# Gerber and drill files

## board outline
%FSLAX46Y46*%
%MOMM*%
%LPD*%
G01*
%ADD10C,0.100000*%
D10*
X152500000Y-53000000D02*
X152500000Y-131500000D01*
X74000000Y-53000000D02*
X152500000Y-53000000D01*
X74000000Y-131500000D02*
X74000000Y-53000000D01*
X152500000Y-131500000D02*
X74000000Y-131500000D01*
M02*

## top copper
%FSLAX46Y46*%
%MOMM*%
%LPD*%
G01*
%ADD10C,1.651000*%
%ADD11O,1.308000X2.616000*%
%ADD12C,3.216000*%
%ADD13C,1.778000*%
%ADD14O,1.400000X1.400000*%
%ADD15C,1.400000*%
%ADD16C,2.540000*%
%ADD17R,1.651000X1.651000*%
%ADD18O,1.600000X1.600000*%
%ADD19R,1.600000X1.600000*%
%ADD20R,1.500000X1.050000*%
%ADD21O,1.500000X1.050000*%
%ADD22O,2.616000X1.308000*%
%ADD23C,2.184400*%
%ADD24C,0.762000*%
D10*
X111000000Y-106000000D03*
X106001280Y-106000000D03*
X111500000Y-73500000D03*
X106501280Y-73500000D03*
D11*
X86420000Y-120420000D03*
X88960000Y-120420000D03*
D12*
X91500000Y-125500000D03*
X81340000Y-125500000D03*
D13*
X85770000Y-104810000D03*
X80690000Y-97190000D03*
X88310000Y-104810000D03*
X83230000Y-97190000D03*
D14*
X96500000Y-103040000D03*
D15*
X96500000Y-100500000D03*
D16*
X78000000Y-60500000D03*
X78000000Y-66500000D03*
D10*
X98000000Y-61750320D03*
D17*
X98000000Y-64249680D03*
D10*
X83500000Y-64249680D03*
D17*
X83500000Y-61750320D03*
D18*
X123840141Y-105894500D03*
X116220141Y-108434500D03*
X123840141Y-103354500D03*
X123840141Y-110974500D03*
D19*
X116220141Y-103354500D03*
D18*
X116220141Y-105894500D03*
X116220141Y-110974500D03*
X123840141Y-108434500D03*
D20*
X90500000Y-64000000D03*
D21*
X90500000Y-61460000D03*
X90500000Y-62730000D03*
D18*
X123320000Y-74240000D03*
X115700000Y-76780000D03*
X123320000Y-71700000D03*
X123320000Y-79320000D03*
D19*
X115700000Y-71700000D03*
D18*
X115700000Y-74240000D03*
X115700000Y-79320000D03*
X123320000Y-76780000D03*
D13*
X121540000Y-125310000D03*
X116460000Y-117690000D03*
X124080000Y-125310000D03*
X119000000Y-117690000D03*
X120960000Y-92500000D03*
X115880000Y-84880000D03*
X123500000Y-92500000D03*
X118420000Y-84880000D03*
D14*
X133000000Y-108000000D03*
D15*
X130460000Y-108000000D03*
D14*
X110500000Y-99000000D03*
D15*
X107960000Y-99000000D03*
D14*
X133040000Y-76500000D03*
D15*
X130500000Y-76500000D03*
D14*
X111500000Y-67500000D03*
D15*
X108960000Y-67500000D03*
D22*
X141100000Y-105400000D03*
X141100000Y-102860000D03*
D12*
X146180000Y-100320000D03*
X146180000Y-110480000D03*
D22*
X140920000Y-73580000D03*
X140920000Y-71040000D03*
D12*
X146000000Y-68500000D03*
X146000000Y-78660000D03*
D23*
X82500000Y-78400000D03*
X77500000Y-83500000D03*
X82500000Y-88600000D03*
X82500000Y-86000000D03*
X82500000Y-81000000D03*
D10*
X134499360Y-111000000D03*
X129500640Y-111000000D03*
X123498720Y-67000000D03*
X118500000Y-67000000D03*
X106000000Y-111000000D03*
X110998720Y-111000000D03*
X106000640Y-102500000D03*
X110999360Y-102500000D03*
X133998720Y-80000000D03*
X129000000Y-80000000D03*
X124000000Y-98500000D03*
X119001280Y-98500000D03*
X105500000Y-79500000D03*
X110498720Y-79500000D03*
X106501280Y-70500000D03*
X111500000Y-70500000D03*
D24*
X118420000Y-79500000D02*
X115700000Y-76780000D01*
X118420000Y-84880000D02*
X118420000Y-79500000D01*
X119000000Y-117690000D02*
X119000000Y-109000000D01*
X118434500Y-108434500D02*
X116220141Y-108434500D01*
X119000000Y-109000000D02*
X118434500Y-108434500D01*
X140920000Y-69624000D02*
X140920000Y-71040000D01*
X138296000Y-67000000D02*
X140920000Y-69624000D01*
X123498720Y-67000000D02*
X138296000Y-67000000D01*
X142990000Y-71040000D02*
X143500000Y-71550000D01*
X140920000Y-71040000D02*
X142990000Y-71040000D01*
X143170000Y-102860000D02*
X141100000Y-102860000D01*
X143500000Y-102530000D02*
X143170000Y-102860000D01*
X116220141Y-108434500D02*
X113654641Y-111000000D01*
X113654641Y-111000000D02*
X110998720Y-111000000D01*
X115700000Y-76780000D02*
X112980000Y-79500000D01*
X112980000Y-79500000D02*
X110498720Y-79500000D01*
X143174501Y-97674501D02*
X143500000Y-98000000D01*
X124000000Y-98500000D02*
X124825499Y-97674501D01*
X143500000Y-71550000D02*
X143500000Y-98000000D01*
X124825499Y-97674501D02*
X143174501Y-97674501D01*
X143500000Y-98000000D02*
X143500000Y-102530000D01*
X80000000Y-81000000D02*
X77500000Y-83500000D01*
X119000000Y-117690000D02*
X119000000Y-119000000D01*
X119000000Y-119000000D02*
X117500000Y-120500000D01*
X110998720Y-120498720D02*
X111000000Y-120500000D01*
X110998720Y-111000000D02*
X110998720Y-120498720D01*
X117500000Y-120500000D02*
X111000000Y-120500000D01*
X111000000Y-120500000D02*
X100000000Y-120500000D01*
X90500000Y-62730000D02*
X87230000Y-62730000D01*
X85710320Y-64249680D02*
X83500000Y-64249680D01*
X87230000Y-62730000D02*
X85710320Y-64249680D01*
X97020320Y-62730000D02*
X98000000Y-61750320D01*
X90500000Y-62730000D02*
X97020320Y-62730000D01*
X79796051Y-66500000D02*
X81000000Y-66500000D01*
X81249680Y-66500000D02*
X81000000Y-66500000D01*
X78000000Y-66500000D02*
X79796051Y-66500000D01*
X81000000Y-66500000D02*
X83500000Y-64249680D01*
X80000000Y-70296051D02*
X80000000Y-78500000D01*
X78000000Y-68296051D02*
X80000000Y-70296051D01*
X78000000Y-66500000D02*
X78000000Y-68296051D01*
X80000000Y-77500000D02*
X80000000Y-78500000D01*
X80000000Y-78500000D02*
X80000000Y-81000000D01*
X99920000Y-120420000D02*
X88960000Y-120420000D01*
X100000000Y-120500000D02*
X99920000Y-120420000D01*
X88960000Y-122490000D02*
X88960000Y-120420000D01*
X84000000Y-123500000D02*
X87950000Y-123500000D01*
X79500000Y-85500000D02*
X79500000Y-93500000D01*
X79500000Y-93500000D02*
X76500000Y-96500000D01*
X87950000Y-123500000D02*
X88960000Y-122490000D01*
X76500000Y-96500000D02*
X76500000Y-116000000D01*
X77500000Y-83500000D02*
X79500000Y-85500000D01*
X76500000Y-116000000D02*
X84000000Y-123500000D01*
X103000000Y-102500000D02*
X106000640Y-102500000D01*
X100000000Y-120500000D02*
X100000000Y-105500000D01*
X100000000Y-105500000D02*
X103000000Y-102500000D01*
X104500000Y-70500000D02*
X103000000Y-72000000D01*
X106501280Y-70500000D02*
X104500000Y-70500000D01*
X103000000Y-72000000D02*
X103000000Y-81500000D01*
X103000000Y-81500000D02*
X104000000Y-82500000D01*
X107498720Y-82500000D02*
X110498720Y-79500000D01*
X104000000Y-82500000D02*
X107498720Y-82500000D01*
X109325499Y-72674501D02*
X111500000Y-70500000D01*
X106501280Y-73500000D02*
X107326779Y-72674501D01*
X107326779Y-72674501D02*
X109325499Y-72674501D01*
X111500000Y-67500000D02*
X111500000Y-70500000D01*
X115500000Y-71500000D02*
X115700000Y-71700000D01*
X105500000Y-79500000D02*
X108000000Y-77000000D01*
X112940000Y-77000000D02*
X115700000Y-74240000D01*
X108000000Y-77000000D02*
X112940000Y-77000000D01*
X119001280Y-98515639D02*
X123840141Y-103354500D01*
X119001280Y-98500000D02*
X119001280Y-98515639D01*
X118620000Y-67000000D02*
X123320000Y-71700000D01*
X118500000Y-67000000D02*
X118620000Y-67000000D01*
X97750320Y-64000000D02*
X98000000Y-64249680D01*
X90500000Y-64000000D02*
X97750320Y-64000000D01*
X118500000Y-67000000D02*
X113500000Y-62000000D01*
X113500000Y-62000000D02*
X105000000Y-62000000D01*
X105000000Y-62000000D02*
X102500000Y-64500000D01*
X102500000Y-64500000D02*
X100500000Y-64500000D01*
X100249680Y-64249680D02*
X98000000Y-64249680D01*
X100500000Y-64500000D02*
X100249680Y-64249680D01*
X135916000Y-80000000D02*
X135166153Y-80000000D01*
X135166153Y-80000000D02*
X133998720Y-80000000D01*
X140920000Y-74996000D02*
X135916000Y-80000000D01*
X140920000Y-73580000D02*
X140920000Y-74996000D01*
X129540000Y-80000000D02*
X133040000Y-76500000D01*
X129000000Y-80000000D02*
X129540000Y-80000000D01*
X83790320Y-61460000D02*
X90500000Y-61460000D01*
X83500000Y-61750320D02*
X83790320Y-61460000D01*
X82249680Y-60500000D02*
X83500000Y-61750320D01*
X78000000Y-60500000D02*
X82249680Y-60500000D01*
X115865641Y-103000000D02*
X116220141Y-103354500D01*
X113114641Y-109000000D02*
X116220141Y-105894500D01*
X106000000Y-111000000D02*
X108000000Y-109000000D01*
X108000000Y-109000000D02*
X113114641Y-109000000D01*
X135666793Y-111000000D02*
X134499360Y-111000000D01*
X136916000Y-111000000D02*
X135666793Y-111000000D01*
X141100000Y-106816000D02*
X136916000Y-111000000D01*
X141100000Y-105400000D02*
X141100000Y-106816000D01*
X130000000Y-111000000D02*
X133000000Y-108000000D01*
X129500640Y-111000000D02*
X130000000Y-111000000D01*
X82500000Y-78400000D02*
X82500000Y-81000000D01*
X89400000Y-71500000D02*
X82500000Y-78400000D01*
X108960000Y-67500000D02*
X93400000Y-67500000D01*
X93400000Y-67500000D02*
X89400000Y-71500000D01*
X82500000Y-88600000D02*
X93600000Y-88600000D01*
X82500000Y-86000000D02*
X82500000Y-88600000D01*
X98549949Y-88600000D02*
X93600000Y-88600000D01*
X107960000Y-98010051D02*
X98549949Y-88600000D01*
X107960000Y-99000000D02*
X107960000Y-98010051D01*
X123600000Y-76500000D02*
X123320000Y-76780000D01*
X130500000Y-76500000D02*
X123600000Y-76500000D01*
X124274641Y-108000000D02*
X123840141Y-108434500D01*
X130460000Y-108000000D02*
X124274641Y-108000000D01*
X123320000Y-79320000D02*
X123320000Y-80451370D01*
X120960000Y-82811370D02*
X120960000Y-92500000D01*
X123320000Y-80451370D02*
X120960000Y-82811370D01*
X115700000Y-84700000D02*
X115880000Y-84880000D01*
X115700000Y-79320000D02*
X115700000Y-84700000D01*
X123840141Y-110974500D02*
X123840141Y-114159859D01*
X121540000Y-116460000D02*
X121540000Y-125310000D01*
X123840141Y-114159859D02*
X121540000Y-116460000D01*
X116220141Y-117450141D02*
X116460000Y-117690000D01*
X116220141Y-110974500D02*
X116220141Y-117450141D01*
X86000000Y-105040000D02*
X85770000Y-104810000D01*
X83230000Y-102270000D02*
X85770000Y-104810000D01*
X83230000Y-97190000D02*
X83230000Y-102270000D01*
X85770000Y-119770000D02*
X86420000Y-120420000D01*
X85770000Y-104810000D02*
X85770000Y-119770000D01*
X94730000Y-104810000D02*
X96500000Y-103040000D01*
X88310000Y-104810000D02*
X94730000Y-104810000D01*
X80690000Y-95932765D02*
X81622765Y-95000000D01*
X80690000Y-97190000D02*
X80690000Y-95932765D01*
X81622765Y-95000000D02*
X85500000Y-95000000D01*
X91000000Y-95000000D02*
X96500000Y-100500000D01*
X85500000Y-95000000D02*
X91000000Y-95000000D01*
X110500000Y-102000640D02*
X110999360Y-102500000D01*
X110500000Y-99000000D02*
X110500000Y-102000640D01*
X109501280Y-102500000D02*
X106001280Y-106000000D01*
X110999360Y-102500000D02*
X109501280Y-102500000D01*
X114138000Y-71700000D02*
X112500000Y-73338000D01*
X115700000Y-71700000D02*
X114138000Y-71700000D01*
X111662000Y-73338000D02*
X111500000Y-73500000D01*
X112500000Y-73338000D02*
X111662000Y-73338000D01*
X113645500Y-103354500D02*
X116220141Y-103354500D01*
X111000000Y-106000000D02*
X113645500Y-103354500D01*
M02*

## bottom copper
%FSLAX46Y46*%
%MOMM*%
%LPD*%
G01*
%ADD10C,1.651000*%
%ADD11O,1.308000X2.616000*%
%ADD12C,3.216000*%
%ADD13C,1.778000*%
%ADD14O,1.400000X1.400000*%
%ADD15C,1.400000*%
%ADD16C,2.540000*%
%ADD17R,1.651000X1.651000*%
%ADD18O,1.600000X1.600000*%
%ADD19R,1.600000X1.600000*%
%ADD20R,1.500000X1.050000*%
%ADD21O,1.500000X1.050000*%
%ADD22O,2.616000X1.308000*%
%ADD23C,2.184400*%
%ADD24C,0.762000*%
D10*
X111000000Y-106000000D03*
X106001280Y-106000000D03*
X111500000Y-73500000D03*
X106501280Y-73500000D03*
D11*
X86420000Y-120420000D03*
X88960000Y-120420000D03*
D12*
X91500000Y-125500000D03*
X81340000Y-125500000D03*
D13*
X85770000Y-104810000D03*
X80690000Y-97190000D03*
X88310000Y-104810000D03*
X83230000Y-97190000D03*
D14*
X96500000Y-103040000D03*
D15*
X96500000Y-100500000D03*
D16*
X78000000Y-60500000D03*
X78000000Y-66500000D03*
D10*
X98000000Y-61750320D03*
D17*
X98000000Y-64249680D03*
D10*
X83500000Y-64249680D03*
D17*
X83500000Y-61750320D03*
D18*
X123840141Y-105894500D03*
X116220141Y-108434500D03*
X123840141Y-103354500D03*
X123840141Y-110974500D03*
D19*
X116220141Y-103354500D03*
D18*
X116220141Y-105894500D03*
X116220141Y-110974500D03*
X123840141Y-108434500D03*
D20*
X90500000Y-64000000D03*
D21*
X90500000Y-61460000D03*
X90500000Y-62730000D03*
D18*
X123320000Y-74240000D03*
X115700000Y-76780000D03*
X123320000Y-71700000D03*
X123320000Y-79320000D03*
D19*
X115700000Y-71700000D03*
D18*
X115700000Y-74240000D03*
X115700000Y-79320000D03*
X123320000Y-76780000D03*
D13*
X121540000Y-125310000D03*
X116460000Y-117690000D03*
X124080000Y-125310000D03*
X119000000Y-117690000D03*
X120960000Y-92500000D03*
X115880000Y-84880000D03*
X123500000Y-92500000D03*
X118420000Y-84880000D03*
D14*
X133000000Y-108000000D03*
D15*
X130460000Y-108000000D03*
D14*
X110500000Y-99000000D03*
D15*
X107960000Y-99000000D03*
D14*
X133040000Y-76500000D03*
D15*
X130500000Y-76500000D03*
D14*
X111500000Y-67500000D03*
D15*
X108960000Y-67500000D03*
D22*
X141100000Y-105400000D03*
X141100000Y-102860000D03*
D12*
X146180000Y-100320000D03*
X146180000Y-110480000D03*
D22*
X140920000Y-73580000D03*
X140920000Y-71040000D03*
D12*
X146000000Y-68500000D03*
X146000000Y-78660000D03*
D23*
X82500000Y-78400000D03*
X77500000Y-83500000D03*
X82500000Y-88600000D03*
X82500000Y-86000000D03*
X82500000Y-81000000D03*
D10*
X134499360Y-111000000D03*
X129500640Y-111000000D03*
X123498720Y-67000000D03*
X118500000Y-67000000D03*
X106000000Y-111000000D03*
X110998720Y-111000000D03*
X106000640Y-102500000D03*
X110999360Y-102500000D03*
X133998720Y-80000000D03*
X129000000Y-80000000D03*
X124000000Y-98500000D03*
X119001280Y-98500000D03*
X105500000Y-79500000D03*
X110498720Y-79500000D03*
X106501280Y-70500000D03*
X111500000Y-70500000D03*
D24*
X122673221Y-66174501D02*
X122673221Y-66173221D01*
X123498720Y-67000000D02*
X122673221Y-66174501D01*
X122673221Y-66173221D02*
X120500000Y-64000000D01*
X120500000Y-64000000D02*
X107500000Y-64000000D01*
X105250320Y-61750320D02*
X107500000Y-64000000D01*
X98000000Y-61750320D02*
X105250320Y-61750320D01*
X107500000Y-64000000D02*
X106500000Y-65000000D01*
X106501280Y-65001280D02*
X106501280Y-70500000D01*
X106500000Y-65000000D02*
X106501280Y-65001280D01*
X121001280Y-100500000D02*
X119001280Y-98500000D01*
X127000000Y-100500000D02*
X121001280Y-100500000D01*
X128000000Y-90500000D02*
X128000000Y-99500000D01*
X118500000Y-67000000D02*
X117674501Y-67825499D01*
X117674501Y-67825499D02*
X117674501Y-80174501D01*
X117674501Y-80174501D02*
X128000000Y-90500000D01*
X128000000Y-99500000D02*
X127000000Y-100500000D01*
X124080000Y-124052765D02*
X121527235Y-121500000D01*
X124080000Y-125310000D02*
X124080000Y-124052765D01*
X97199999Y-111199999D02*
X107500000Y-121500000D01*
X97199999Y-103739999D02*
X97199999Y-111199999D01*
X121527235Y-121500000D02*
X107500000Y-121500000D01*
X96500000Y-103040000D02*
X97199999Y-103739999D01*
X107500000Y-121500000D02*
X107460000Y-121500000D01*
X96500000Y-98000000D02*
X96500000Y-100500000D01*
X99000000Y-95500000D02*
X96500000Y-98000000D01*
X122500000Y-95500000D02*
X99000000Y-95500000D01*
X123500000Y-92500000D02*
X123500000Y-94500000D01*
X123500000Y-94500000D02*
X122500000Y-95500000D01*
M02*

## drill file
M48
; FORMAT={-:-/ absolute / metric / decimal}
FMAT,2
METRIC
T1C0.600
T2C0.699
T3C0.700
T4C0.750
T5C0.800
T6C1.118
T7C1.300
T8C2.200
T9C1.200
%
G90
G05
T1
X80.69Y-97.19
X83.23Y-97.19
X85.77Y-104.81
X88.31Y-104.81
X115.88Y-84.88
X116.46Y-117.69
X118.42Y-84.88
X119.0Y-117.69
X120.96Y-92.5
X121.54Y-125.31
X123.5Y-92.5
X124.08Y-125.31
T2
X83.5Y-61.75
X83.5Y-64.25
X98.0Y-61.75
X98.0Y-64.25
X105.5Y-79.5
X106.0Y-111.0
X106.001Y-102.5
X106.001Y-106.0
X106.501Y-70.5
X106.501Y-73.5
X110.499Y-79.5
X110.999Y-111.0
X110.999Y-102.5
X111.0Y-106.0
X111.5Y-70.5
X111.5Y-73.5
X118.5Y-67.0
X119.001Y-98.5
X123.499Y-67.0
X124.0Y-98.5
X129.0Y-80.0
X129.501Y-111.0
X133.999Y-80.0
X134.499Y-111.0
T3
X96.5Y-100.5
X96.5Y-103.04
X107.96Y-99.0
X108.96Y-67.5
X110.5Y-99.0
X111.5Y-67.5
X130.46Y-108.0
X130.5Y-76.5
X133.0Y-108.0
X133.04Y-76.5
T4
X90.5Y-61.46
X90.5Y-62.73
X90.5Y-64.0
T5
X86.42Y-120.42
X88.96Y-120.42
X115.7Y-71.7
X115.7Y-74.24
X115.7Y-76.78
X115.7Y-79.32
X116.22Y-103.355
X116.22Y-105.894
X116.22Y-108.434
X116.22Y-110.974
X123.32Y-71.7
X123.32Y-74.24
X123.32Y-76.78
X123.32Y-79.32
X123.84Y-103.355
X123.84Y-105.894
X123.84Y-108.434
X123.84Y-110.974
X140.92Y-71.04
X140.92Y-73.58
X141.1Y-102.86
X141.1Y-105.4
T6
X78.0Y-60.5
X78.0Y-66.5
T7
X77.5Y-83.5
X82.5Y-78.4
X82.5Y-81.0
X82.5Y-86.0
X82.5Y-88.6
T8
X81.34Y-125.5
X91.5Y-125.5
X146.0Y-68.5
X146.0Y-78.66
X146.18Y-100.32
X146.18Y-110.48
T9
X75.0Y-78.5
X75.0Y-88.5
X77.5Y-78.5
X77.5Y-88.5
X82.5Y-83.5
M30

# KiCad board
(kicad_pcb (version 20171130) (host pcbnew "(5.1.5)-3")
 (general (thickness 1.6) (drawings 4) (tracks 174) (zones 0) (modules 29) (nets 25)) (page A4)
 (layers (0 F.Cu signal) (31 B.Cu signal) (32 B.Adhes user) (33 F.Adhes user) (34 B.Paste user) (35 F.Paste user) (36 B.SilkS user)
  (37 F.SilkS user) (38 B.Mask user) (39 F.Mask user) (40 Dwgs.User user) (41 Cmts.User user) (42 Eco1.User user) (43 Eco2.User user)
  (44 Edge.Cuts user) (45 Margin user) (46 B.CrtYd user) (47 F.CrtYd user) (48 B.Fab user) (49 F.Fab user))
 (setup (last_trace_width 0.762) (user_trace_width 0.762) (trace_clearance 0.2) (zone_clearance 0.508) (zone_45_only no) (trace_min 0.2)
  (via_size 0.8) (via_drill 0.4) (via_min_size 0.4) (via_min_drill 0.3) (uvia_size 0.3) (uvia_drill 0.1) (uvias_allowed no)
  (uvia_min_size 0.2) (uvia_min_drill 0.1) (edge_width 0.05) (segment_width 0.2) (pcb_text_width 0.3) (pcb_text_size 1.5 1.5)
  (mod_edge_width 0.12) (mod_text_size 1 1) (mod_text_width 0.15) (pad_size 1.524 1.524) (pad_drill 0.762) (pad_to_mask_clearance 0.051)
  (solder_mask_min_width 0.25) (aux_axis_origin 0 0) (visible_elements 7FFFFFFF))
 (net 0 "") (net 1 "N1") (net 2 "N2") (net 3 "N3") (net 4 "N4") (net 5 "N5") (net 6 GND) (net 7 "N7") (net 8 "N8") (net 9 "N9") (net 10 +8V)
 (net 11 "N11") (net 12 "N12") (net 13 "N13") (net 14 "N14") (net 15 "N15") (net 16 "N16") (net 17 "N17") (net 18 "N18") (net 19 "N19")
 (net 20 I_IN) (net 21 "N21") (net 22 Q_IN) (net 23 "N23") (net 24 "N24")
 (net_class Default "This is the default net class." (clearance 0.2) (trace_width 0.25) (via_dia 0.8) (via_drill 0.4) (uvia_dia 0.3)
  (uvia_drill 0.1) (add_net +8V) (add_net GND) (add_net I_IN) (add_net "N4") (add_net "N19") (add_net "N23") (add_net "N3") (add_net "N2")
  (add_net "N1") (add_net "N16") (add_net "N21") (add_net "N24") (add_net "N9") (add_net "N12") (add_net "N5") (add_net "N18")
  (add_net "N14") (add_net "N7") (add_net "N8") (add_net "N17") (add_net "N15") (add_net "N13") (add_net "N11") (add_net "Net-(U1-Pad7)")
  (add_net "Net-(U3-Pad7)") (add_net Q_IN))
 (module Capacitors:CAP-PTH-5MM (layer F.Cu) (at 108.50064 106)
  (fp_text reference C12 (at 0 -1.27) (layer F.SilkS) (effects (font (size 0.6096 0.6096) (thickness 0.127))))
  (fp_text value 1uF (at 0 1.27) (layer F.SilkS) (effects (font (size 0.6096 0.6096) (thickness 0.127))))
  (pad 2 thru_hole circle (at 2.49936 0) (size 1.651 1.651) (drill 0.6985) (layers *.Cu *.Mask) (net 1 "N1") (solder_mask_margin 0.1016))
  (pad 1 thru_hole circle (at -2.49936 0) (size 1.651 1.651) (drill 0.6985) (layers *.Cu *.Mask) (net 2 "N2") (solder_mask_margin 0.1016)))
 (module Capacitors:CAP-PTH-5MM (layer F.Cu) (at 109.00064 73.5)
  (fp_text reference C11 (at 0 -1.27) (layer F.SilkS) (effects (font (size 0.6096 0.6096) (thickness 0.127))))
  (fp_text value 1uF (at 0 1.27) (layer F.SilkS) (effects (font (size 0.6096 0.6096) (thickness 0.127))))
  (pad 2 thru_hole circle (at 2.49936 0) (size 1.651 1.651) (drill 0.6985) (layers *.Cu *.Mask) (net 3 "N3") (solder_mask_margin 0.1016))
  (pad 1 thru_hole circle (at -2.49936 0) (size 1.651 1.651) (drill 0.6985) (layers *.Cu *.Mask) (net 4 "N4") (solder_mask_margin 0.1016)))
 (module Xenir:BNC (layer F.Cu) (at 86.32 124.32 180)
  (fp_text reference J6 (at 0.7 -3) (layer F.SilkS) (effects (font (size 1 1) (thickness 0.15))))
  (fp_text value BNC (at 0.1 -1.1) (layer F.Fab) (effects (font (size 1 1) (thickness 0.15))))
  (pad S thru_hole oval (at -0.1 3.9 270) (size 2.616 1.308) (drill 0.8) (layers *.Cu *.Mask) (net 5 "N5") (solder_mask_margin 0.1016))
  (pad GND thru_hole oval (at -2.64 3.9 270) (size 2.616 1.308) (drill 0.8) (layers *.Cu *.Mask) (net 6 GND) (solder_mask_margin 0.1016))
  (pad 3 thru_hole circle (at -5.18 -1.18 180) (size 3.216 3.216) (drill 2.2) (layers *.Cu *.Mask) (solder_mask_margin 0.1016))
  (pad 4 thru_hole circle (at 4.98 -1.18 180) (size 3.216 3.216) (drill 2.2) (layers *.Cu *.Mask) (solder_mask_margin 0.1016)))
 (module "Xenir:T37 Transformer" (layer F.Cu) (at 91.5 101 270)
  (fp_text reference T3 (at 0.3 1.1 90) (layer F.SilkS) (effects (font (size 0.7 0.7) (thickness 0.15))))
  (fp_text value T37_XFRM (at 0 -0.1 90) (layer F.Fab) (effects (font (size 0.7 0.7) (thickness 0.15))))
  (pad C1B thru_hole circle (at 3.81 5.73 270) (size 1.778 1.778) (drill 0.6) (layers *.Cu *.Mask) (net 5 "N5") (solder_mask_margin 0.1016))
  (pad C1A thru_hole circle (at -3.81 10.81 270) (size 1.778 1.778) (drill 0.6) (layers *.Cu *.Mask) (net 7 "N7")
   (solder_mask_margin 0.1016))
  (pad C2B thru_hole circle (at 3.81 3.19 270) (size 1.778 1.778) (drill 0.6) (layers *.Cu *.Mask) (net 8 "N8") (solder_mask_margin 0.1016))
  (pad C2A thru_hole circle (at -3.81 8.27 270) (size 1.778 1.778) (drill 0.6) (layers *.Cu *.Mask) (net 5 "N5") (solder_mask_margin 0.1016)))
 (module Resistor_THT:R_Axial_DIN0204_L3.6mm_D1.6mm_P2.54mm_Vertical (layer F.Cu) (at 96.5 100.5 270)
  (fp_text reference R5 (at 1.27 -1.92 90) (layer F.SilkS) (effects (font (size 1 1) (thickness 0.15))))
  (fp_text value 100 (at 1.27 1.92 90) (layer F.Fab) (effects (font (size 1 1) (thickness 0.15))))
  (pad 2 thru_hole oval (at 2.54 0 270) (size 1.4 1.4) (drill 0.7) (layers *.Cu *.Mask) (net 8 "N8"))
  (pad 1 thru_hole circle (at 0 0 270) (size 1.4 1.4) (drill 0.7) (layers *.Cu *.Mask) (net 7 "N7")))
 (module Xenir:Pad (layer F.Cu) (at 78 57)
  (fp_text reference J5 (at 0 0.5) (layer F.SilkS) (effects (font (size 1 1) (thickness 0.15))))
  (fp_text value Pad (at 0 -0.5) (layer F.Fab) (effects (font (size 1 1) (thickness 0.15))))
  (pad 1 thru_hole circle (at 0 3.5) (size 2.54 2.54) (drill 1.1176) (layers *.Cu *.Mask) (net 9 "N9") (solder_mask_margin 0.1016)))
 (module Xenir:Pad (layer F.Cu) (at 78 63)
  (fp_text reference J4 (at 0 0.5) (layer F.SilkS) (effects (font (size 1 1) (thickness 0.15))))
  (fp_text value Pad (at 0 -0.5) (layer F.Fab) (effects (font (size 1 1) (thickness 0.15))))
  (pad 1 thru_hole circle (at 0 3.5) (size 2.54 2.54) (drill 1.1176) (layers *.Cu *.Mask) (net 6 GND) (solder_mask_margin 0.1016)))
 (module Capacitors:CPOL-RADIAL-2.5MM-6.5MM (layer F.Cu) (at 98 63 270)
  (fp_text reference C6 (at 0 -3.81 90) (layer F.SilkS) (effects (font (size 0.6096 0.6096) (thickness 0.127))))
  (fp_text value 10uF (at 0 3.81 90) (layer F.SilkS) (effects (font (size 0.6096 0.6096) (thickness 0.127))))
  (pad 2 thru_hole circle (at -1.24968 0 270) (size 1.651 1.651) (drill 0.6985) (layers *.Cu *.Mask) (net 6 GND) (solder_mask_margin 0.1016))
  (pad 1 thru_hole rect (at 1.24968 0 270) (size 1.651 1.651) (drill 0.6985) (layers *.Cu *.Mask) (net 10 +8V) (solder_mask_margin 0.1016)))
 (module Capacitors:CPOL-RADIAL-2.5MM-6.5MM (layer F.Cu) (at 83.5 63 90)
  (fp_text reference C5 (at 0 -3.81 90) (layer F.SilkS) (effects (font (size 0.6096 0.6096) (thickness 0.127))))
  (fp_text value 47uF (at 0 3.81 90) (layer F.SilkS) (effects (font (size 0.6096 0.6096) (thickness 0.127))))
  (pad 2 thru_hole circle (at -1.24968 0 90) (size 1.651 1.651) (drill 0.6985) (layers *.Cu *.Mask) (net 6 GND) (solder_mask_margin 0.1016))
  (pad 1 thru_hole rect (at 1.24968 0 90) (size 1.651 1.651) (drill 0.6985) (layers *.Cu *.Mask) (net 9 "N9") (solder_mask_margin 0.1016)))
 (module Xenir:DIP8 (layer F.Cu) (at 120.020141 101.6545)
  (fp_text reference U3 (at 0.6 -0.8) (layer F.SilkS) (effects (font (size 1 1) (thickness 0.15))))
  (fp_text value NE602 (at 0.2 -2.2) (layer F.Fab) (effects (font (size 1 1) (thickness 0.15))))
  (pad 7 thru_hole oval (at 3.82 4.24) (size 1.6 1.6) (drill 0.8) (layers *.Cu *.Mask))
  (pad 3 thru_hole oval (at -3.8 6.78) (size 1.6 1.6) (drill 0.8) (layers *.Cu *.Mask) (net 6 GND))
  (pad 8 thru_hole oval (at 3.82 1.7) (size 1.6 1.6) (drill 0.8) (layers *.Cu *.Mask) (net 10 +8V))
  (pad 5 thru_hole oval (at 3.82 9.32) (size 1.6 1.6) (drill 0.8) (layers *.Cu *.Mask) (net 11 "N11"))
  (pad 1 thru_hole rect (at -3.8 1.7) (size 1.6 1.6) (drill 0.8) (layers *.Cu *.Mask) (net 1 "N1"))
  (pad 2 thru_hole oval (at -3.8 4.24) (size 1.6 1.6) (drill 0.8) (layers *.Cu *.Mask) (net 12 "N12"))
  (pad 4 thru_hole oval (at -3.8 9.32) (size 1.6 1.6) (drill 0.8) (layers *.Cu *.Mask) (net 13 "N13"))
  (pad 6 thru_hole oval (at 3.82 6.78) (size 1.6 1.6) (drill 0.8) (layers *.Cu *.Mask) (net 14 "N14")))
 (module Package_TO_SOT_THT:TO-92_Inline (layer F.Cu) (at 90.5 64 90)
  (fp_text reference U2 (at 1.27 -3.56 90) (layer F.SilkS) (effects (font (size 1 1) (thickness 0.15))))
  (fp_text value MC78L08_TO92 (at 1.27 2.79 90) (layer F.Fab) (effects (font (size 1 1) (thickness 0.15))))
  (pad 1 thru_hole rect (at 0 0 90) (size 1.05 1.5) (drill 0.75) (layers *.Cu *.Mask) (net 10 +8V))
  (pad 3 thru_hole oval (at 2.54 0 90) (size 1.05 1.5) (drill 0.75) (layers *.Cu *.Mask) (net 9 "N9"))
  (pad 2 thru_hole oval (at 1.27 0 90) (size 1.05 1.5) (drill 0.75) (layers *.Cu *.Mask) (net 6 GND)))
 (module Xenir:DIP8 (layer F.Cu) (at 119.5 70)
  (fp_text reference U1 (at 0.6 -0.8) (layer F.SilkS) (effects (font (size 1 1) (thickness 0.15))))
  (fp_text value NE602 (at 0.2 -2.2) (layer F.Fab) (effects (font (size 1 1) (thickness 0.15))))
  (pad 7 thru_hole oval (at 3.82 4.24) (size 1.6 1.6) (drill 0.8) (layers *.Cu *.Mask))
  (pad 3 thru_hole oval (at -3.8 6.78) (size 1.6 1.6) (drill 0.8) (layers *.Cu *.Mask) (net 6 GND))
  (pad 8 thru_hole oval (at 3.82 1.7) (size 1.6 1.6) (drill 0.8) (layers *.Cu *.Mask) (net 10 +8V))
  (pad 5 thru_hole oval (at 3.82 9.32) (size 1.6 1.6) (drill 0.8) (layers *.Cu *.Mask) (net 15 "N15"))
  (pad 1 thru_hole rect (at -3.8 1.7) (size 1.6 1.6) (drill 0.8) (layers *.Cu *.Mask) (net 3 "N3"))
  (pad 2 thru_hole oval (at -3.8 4.24) (size 1.6 1.6) (drill 0.8) (layers *.Cu *.Mask) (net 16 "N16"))
  (pad 4 thru_hole oval (at -3.8 9.32) (size 1.6 1.6) (drill 0.8) (layers *.Cu *.Mask) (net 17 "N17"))
  (pad 6 thru_hole oval (at 3.82 6.78) (size 1.6 1.6) (drill 0.8) (layers *.Cu *.Mask) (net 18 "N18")))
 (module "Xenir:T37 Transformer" (layer F.Cu) (at 127.27 121.5 270)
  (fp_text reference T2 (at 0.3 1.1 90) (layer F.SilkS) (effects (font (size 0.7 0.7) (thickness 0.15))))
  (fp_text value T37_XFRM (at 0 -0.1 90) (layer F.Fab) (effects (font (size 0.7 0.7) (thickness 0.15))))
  (pad C1B thru_hole circle (at 3.81 5.73 270) (size 1.778 1.778) (drill 0.6) (layers *.Cu *.Mask) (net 11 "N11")
   (solder_mask_margin 0.1016))
  (pad C1A thru_hole circle (at -3.81 10.81 270) (size 1.778 1.778) (drill 0.6) (layers *.Cu *.Mask) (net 13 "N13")
   (solder_mask_margin 0.1016))
  (pad C2B thru_hole circle (at 3.81 3.19 270) (size 1.778 1.778) (drill 0.6) (layers *.Cu *.Mask) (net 8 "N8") (solder_mask_margin 0.1016))
  (pad C2A thru_hole circle (at -3.81 8.27 270) (size 1.778 1.778) (drill 0.6) (layers *.Cu *.Mask) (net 6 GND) (solder_mask_margin 0.1016)))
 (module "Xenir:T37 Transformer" (layer F.Cu) (at 126.69 88.69 270)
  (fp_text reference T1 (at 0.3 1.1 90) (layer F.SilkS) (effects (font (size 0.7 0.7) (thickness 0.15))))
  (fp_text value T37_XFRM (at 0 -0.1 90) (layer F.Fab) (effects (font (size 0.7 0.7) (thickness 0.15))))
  (pad C1B thru_hole circle (at 3.81 5.73 270) (size 1.778 1.778) (drill 0.6) (layers *.Cu *.Mask) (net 15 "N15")
   (solder_mask_margin 0.1016))
  (pad C1A thru_hole circle (at -3.81 10.81 270) (size 1.778 1.778) (drill 0.6) (layers *.Cu *.Mask) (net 17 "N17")
   (solder_mask_margin 0.1016))
  (pad C2B thru_hole circle (at 3.81 3.19 270) (size 1.778 1.778) (drill 0.6) (layers *.Cu *.Mask) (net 7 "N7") (solder_mask_margin 0.1016))
  (pad C2A thru_hole circle (at -3.81 8.27 270) (size 1.778 1.778) (drill 0.6) (layers *.Cu *.Mask) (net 6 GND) (solder_mask_margin 0.1016)))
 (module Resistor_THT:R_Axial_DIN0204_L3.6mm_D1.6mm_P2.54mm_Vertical (layer F.Cu) (at 130.46 108)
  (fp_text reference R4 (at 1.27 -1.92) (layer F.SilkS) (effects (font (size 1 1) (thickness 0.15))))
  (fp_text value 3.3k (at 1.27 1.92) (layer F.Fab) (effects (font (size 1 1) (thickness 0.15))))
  (pad 2 thru_hole oval (at 2.54 0) (size 1.4 1.4) (drill 0.7) (layers *.Cu *.Mask) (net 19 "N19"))
  (pad 1 thru_hole circle (at 0 0) (size 1.4 1.4) (drill 0.7) (layers *.Cu *.Mask) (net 14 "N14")))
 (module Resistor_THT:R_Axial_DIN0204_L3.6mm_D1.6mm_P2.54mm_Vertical (layer F.Cu) (at 107.96 99)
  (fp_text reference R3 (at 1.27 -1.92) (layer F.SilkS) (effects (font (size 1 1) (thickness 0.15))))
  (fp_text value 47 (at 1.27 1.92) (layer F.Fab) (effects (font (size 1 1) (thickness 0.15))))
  (pad 2 thru_hole oval (at 2.54 0) (size 1.4 1.4) (drill 0.7) (layers *.Cu *.Mask) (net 2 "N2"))
  (pad 1 thru_hole circle (at 0 0) (size 1.4 1.4) (drill 0.7) (layers *.Cu *.Mask) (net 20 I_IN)))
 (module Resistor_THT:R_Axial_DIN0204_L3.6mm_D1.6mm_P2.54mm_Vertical (layer F.Cu) (at 130.5 76.5)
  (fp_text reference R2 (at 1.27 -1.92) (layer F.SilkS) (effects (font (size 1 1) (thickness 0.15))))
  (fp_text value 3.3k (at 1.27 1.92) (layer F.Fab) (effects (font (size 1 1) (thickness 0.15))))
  (pad 2 thru_hole oval (at 2.54 0) (size 1.4 1.4) (drill 0.7) (layers *.Cu *.Mask) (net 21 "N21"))
  (pad 1 thru_hole circle (at 0 0) (size 1.4 1.4) (drill 0.7) (layers *.Cu *.Mask) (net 18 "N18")))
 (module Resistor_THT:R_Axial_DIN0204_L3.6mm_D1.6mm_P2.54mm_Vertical (layer F.Cu) (at 108.96 67.5)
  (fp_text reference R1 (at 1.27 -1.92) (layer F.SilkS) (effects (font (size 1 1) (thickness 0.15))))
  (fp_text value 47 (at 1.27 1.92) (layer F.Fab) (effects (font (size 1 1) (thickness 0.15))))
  (pad 2 thru_hole oval (at 2.54 0) (size 1.4 1.4) (drill 0.7) (layers *.Cu *.Mask) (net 4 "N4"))
  (pad 1 thru_hole circle (at 0 0) (size 1.4 1.4) (drill 0.7) (layers *.Cu *.Mask) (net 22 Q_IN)))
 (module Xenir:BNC (layer F.Cu) (at 145 105.5 270)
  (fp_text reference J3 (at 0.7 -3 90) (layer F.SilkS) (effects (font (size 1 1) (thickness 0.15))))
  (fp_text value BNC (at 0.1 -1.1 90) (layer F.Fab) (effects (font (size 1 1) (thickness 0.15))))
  (pad S thru_hole oval (at -0.1 3.9) (size 2.616 1.308) (drill 0.8) (layers *.Cu *.Mask) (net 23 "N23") (solder_mask_margin 0.1016))
  (pad GND thru_hole oval (at -2.64 3.9) (size 2.616 1.308) (drill 0.8) (layers *.Cu *.Mask) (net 6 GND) (solder_mask_margin 0.1016))
  (pad 3 thru_hole circle (at -5.18 -1.18 270) (size 3.216 3.216) (drill 2.2) (layers *.Cu *.Mask) (solder_mask_margin 0.1016))
  (pad 4 thru_hole circle (at 4.98 -1.18 270) (size 3.216 3.216) (drill 2.2) (layers *.Cu *.Mask) (solder_mask_margin 0.1016)))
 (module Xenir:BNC (layer F.Cu) (at 144.82 73.68 270)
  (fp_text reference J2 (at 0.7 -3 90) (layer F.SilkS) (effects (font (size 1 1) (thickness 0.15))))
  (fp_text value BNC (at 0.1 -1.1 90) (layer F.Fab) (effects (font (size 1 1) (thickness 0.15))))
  (pad S thru_hole oval (at -0.1 3.9) (size 2.616 1.308) (drill 0.8) (layers *.Cu *.Mask) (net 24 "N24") (solder_mask_margin 0.1016))
  (pad GND thru_hole oval (at -2.64 3.9) (size 2.616 1.308) (drill 0.8) (layers *.Cu *.Mask) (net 6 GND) (solder_mask_margin 0.1016))
  (pad 3 thru_hole circle (at -5.18 -1.18 270) (size 3.216 3.216) (drill 2.2) (layers *.Cu *.Mask) (solder_mask_margin 0.1016))
  (pad 4 thru_hole circle (at 4.98 -1.18 270) (size 3.216 3.216) (drill 2.2) (layers *.Cu *.Mask) (solder_mask_margin 0.1016)))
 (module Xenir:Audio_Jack (layer F.Cu) (at 79.5 75)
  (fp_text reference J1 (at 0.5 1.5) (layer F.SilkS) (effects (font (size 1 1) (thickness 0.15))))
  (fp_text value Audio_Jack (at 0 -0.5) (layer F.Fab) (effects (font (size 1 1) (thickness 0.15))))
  (pad "" np_thru_hole circle (at -4.5 3.5) (size 1.2 1.2) (drill 1.2) (layers *.Cu *.Mask))
  (pad "" np_thru_hole circle (at -2 3.5) (size 1.2 1.2) (drill 1.2) (layers *.Cu *.Mask))
  (pad RING thru_hole circle (at 3 3.4) (size 2.1844 2.1844) (drill 1.3) (layers *.Cu *.Mask) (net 22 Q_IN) (solder_mask_margin 0.1016))
  (pad "" np_thru_hole circle (at 3 8.5) (size 1.2 1.2) (drill 1.2) (layers *.Cu *.Mask))
  (pad SLEEVE thru_hole circle (at -2 8.5) (size 2.1844 2.1844) (drill 1.3) (layers *.Cu *.Mask) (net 6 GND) (solder_mask_margin 0.1016))
  (pad "" np_thru_hole circle (at -2 13.5) (size 1.2 1.2) (drill 1.2) (layers *.Cu *.Mask))
  (pad TIP thru_hole circle (at 3 13.6) (size 2.1844 2.1844) (drill 1.3) (layers *.Cu *.Mask) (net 20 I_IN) (solder_mask_margin 0.1016))
  (pad TSH thru_hole circle (at 3 11) (size 2.1844 2.1844) (drill 1.3) (layers *.Cu *.Mask) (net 20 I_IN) (solder_mask_margin 0.1016))
  (pad "" np_thru_hole circle (at -4.5 13.5) (size 1.2 1.2) (drill 1.2) (layers *.Cu *.Mask))
  (pad RSH thru_hole circle (at 3 6) (size 2.1844 2.1844) (drill 1.3) (layers *.Cu *.Mask) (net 22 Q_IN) (solder_mask_margin 0.1016)))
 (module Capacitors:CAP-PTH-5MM (layer F.Cu) (at 132 111)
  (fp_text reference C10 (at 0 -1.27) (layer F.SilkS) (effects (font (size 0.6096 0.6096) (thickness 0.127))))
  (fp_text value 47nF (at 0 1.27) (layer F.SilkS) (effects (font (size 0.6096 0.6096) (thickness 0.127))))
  (pad 2 thru_hole circle (at 2.49936 0) (size 1.651 1.651) (drill 0.6985) (layers *.Cu *.Mask) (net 23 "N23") (solder_mask_margin 0.1016))
  (pad 1 thru_hole circle (at -2.49936 0) (size 1.651 1.651) (drill 0.6985) (layers *.Cu *.Mask) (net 19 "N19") (solder_mask_margin 0.1016)))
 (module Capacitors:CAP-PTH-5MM (layer F.Cu) (at 120.99936 67)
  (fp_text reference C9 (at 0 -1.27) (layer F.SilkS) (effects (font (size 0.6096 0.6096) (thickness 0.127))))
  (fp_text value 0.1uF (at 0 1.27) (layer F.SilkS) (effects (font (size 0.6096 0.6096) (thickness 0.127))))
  (pad 2 thru_hole circle (at 2.49936 0) (size 1.651 1.651) (drill 0.6985) (layers *.Cu *.Mask) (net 6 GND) (solder_mask_margin 0.1016))
  (pad 1 thru_hole circle (at -2.49936 0) (size 1.651 1.651) (drill 0.6985) (layers *.Cu *.Mask) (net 10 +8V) (solder_mask_margin 0.1016)))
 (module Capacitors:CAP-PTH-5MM (layer F.Cu) (at 108.49936 111 180)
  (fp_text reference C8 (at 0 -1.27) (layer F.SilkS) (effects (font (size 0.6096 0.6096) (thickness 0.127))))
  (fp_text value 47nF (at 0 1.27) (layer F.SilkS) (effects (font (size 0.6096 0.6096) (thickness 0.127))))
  (pad 2 thru_hole circle (at 2.49936 0 180) (size 1.651 1.651) (drill 0.6985) (layers *.Cu *.Mask) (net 12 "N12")
   (solder_mask_margin 0.1016))
  (pad 1 thru_hole circle (at -2.49936 0 180) (size 1.651 1.651) (drill 0.6985) (layers *.Cu *.Mask) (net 6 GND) (solder_mask_margin 0.1016)))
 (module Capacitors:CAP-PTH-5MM (layer F.Cu) (at 108.5 102.5 180)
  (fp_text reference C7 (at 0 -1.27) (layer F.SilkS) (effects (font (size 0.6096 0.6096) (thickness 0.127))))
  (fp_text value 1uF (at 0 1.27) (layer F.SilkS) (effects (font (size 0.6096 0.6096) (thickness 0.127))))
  (pad 2 thru_hole circle (at 2.49936 0 180) (size 1.651 1.651) (drill 0.6985) (layers *.Cu *.Mask) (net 6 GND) (solder_mask_margin 0.1016))
  (pad 1 thru_hole circle (at -2.49936 0 180) (size 1.651 1.651) (drill 0.6985) (layers *.Cu *.Mask) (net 2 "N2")
   (solder_mask_margin 0.1016)))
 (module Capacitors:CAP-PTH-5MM (layer F.Cu) (at 131.49936 80)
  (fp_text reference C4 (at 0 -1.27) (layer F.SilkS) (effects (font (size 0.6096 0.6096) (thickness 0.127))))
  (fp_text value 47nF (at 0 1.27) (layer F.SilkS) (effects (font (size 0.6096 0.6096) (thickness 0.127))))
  (pad 2 thru_hole circle (at 2.49936 0) (size 1.651 1.651) (drill 0.6985) (layers *.Cu *.Mask) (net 24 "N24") (solder_mask_margin 0.1016))
  (pad 1 thru_hole circle (at -2.49936 0) (size 1.651 1.651) (drill 0.6985) (layers *.Cu *.Mask) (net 21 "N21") (solder_mask_margin 0.1016)))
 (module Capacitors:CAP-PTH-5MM (layer F.Cu) (at 121.50064 98.5)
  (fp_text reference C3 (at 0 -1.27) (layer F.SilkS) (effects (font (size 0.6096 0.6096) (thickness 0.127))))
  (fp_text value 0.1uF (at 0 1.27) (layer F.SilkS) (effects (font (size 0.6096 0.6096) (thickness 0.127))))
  (pad 2 thru_hole circle (at 2.49936 0) (size 1.651 1.651) (drill 0.6985) (layers *.Cu *.Mask) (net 6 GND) (solder_mask_margin 0.1016))
  (pad 1 thru_hole circle (at -2.49936 0) (size 1.651 1.651) (drill 0.6985) (layers *.Cu *.Mask) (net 10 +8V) (solder_mask_margin 0.1016)))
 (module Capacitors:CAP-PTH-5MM (layer F.Cu) (at 107.99936 79.5 180)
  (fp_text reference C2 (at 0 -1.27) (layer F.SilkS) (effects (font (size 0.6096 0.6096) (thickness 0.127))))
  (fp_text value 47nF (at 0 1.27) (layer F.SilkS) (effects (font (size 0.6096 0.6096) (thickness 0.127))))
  (pad 2 thru_hole circle (at 2.49936 0 180) (size 1.651 1.651) (drill 0.6985) (layers *.Cu *.Mask) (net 16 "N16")
   (solder_mask_margin 0.1016))
  (pad 1 thru_hole circle (at -2.49936 0 180) (size 1.651 1.651) (drill 0.6985) (layers *.Cu *.Mask) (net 6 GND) (solder_mask_margin 0.1016)))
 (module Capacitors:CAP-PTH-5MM (layer F.Cu) (at 109.00064 70.5 180)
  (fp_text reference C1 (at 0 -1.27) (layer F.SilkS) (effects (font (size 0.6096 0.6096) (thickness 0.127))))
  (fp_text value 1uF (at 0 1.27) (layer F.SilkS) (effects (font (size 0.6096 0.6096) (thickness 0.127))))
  (pad 2 thru_hole circle (at 2.49936 0 180) (size 1.651 1.651) (drill 0.6985) (layers *.Cu *.Mask) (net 6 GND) (solder_mask_margin 0.1016))
  (pad 1 thru_hole circle (at -2.49936 0 180) (size 1.651 1.651) (drill 0.6985) (layers *.Cu *.Mask) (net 4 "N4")
   (solder_mask_margin 0.1016)))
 (gr_line (start 152.5 53) (end 152.5 131.5) (layer Edge.Cuts) (width 0.1))
 (gr_line (start 74 53) (end 152.5 53) (layer Edge.Cuts) (width 0.1))
 (gr_line (start 74 131.5) (end 74 53) (layer Edge.Cuts) (width 0.1))
 (gr_line (start 152.5 131.5) (end 74 131.5) (layer Edge.Cuts) (width 0.1))
 (segment (start 118.42 79.5) (end 115.7 76.78) (width 0.762) (layer F.Cu) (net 6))
 (segment (start 118.42 84.88) (end 118.42 79.5) (width 0.762) (layer F.Cu) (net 6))
 (segment (start 119 117.69) (end 119 109) (width 0.762) (layer F.Cu) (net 6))
 (segment (start 118.4345 108.4345) (end 116.220141 108.4345) (width 0.762) (layer F.Cu) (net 6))
 (segment (start 119 109) (end 118.4345 108.4345) (width 0.762) (layer F.Cu) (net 6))
 (segment (start 140.92 69.624) (end 140.92 71.04) (width 0.762) (layer F.Cu) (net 6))
 (segment (start 138.296 67) (end 140.92 69.624) (width 0.762) (layer F.Cu) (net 6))
 (segment (start 123.49872 67) (end 138.296 67) (width 0.762) (layer F.Cu) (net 6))
 (segment (start 142.99 71.04) (end 143.5 71.55) (width 0.762) (layer F.Cu) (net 6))
 (segment (start 140.92 71.04) (end 142.99 71.04) (width 0.762) (layer F.Cu) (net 6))
 (segment (start 143.17 102.86) (end 141.1 102.86) (width 0.762) (layer F.Cu) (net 6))
 (segment (start 143.5 102.53) (end 143.17 102.86) (width 0.762) (layer F.Cu) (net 6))
 (segment (start 116.220141 108.4345) (end 113.654641 111) (width 0.762) (layer F.Cu) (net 6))
 (segment (start 113.654641 111) (end 110.99872 111) (width 0.762) (layer F.Cu) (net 6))
 (segment (start 115.7 76.78) (end 112.98 79.5) (width 0.762) (layer F.Cu) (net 6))
 (segment (start 112.98 79.5) (end 110.49872 79.5) (width 0.762) (layer F.Cu) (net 6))
 (segment (start 143.174501 97.674501) (end 143.5 98) (width 0.762) (layer F.Cu) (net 6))
 (segment (start 124 98.5) (end 124.825499 97.674501) (width 0.762) (layer F.Cu) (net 6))
 (segment (start 143.5 71.55) (end 143.5 98) (width 0.762) (layer F.Cu) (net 6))
 (segment (start 124.825499 97.674501) (end 143.174501 97.674501) (width 0.762) (layer F.Cu) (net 6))
 (segment (start 143.5 98) (end 143.5 102.53) (width 0.762) (layer F.Cu) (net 6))
 (segment (start 80 81) (end 77.5 83.5) (width 0.762) (layer F.Cu) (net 6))
 (segment (start 119 117.69) (end 119 119) (width 0.762) (layer F.Cu) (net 6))
 (segment (start 119 119) (end 117.5 120.5) (width 0.762) (layer F.Cu) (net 6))
 (segment (start 110.99872 120.49872) (end 111 120.5) (width 0.762) (layer F.Cu) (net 6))
 (segment (start 110.99872 111) (end 110.99872 120.49872) (width 0.762) (layer F.Cu) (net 6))
 (segment (start 117.5 120.5) (end 111 120.5) (width 0.762) (layer F.Cu) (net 6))
 (segment (start 111 120.5) (end 100 120.5) (width 0.762) (layer F.Cu) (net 6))
 (segment (start 122.673221 66.174501) (end 122.673221 66.173221) (width 0.762) (layer B.Cu) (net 6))
 (segment (start 123.49872 67) (end 122.673221 66.174501) (width 0.762) (layer B.Cu) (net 6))
 (segment (start 122.673221 66.173221) (end 120.5 64) (width 0.762) (layer B.Cu) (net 6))
 (segment (start 120.5 64) (end 107.5 64) (width 0.762) (layer B.Cu) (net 6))
 (segment (start 105.25032 61.75032) (end 107.5 64) (width 0.762) (layer B.Cu) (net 6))
 (segment (start 98 61.75032) (end 105.25032 61.75032) (width 0.762) (layer B.Cu) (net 6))
 (segment (start 90.5 62.73) (end 87.23 62.73) (width 0.762) (layer F.Cu) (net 6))
 (segment (start 85.71032 64.24968) (end 83.5 64.24968) (width 0.762) (layer F.Cu) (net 6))
 (segment (start 87.23 62.73) (end 85.71032 64.24968) (width 0.762) (layer F.Cu) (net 6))
 (segment (start 97.02032 62.73) (end 98 61.75032) (width 0.762) (layer F.Cu) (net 6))
 (segment (start 90.5 62.73) (end 97.02032 62.73) (width 0.762) (layer F.Cu) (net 6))
 (segment (start 79.796051 66.5) (end 81 66.5) (width 0.762) (layer F.Cu) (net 6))
 (segment (start 81.24968 66.5) (end 81 66.5) (width 0.762) (layer F.Cu) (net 6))
 (segment (start 78 66.5) (end 79.796051 66.5) (width 0.762) (layer F.Cu) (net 6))
 (segment (start 81 66.5) (end 83.5 64.24968) (width 0.762) (layer F.Cu) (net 6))
 (segment (start 80 70.296051) (end 80 78.5) (width 0.762) (layer F.Cu) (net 6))
 (segment (start 78 68.296051) (end 80 70.296051) (width 0.762) (layer F.Cu) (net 6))
 (segment (start 78 66.5) (end 78 68.296051) (width 0.762) (layer F.Cu) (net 6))
 (segment (start 80 77.5) (end 80 78.5) (width 0.762) (layer F.Cu) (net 6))
 (segment (start 80 78.5) (end 80 81) (width 0.762) (layer F.Cu) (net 6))
 (segment (start 99.92 120.42) (end 88.96 120.42) (width 0.762) (layer F.Cu) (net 6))
 (segment (start 100 120.5) (end 99.92 120.42) (width 0.762) (layer F.Cu) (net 6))
 (segment (start 88.96 122.49) (end 88.96 120.42) (width 0.762) (layer F.Cu) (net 6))
 (segment (start 84 123.5) (end 87.95 123.5) (width 0.762) (layer F.Cu) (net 6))
 (segment (start 79.5 85.5) (end 79.5 93.5) (width 0.762) (layer F.Cu) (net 6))
 (segment (start 79.5 93.5) (end 76.5 96.5) (width 0.762) (layer F.Cu) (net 6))
 (segment (start 87.95 123.5) (end 88.96 122.49) (width 0.762) (layer F.Cu) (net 6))
 (segment (start 76.5 96.5) (end 76.5 116) (width 0.762) (layer F.Cu) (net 6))
 (segment (start 77.5 83.5) (end 79.5 85.5) (width 0.762) (layer F.Cu) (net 6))
 (segment (start 76.5 116) (end 84 123.5) (width 0.762) (layer F.Cu) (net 6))
 (segment (start 103 102.5) (end 106.00064 102.5) (width 0.762) (layer F.Cu) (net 6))
 (segment (start 100 120.5) (end 100 105.5) (width 0.762) (layer F.Cu) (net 6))
 (segment (start 100 105.5) (end 103 102.5) (width 0.762) (layer F.Cu) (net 6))
 (segment (start 104.5 70.5) (end 103 72) (width 0.762) (layer F.Cu) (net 6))
 (segment (start 106.50128 70.5) (end 104.5 70.5) (width 0.762) (layer F.Cu) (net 6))
 (segment (start 103 72) (end 103 81.5) (width 0.762) (layer F.Cu) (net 6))
 (segment (start 103 81.5) (end 104 82.5) (width 0.762) (layer F.Cu) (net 6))
 (segment (start 107.49872 82.5) (end 110.49872 79.5) (width 0.762) (layer F.Cu) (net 6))
 (segment (start 104 82.5) (end 107.49872 82.5) (width 0.762) (layer F.Cu) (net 6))
 (segment (start 107.5 64) (end 106.5 65) (width 0.762) (layer B.Cu) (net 6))
 (segment (start 106.50128 65.00128) (end 106.50128 70.5) (width 0.762) (layer B.Cu) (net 6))
 (segment (start 106.5 65) (end 106.50128 65.00128) (width 0.762) (layer B.Cu) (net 6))
 (segment (start 109.325499 72.674501) (end 111.5 70.5) (width 0.762) (layer F.Cu) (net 4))
 (segment (start 106.50128 73.5) (end 107.326779 72.674501) (width 0.762) (layer F.Cu) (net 4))
 (segment (start 107.326779 72.674501) (end 109.325499 72.674501) (width 0.762) (layer F.Cu) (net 4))
 (segment (start 111.5 67.5) (end 111.5 70.5) (width 0.762) (layer F.Cu) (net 4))
 (segment (start 115.5 71.5) (end 115.7 71.7) (width 0.762) (layer F.Cu) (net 3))
 (segment (start 105.5 79.5) (end 108 77) (width 0.762) (layer F.Cu) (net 16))
 (segment (start 112.94 77) (end 115.7 74.24) (width 0.762) (layer F.Cu) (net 16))
 (segment (start 108 77) (end 112.94 77) (width 0.762) (layer F.Cu) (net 16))
 (segment (start 119.00128 98.515639) (end 123.840141 103.3545) (width 0.762) (layer F.Cu) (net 10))
 (segment (start 119.00128 98.5) (end 119.00128 98.515639) (width 0.762) (layer F.Cu) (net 10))
 (segment (start 118.62 67) (end 123.32 71.7) (width 0.762) (layer F.Cu) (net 10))
 (segment (start 118.5 67) (end 118.62 67) (width 0.762) (layer F.Cu) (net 10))
 (segment (start 121.00128 100.5) (end 119.00128 98.5) (width 0.762) (layer B.Cu) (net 10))
 (segment (start 127 100.5) (end 121.00128 100.5) (width 0.762) (layer B.Cu) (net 10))
 (segment (start 128 90.5) (end 128 99.5) (width 0.762) (layer B.Cu) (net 10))
 (segment (start 118.5 67) (end 117.674501 67.825499) (width 0.762) (layer B.Cu) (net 10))
 (segment (start 117.674501 67.825499) (end 117.674501 80.174501) (width 0.762) (layer B.Cu) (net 10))
 (segment (start 117.674501 80.174501) (end 128 90.5) (width 0.762) (layer B.Cu) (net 10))
 (segment (start 128 99.5) (end 127 100.5) (width 0.762) (layer B.Cu) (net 10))
 (segment (start 97.75032 64) (end 98 64.24968) (width 0.762) (layer F.Cu) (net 10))
 (segment (start 90.5 64) (end 97.75032 64) (width 0.762) (layer F.Cu) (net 10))
 (segment (start 118.5 67) (end 113.5 62) (width 0.762) (layer F.Cu) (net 10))
 (segment (start 113.5 62) (end 105 62) (width 0.762) (layer F.Cu) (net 10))
 (segment (start 105 62) (end 102.5 64.5) (width 0.762) (layer F.Cu) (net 10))
 (segment (start 102.5 64.5) (end 100.5 64.5) (width 0.762) (layer F.Cu) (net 10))
 (segment (start 100.24968 64.24968) (end 98 64.24968) (width 0.762) (layer F.Cu) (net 10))
 (segment (start 100.5 64.5) (end 100.24968 64.24968) (width 0.762) (layer F.Cu) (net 10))
 (segment (start 135.916 80) (end 135.166153 80) (width 0.762) (layer F.Cu) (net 24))
 (segment (start 135.166153 80) (end 133.99872 80) (width 0.762) (layer F.Cu) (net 24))
 (segment (start 140.92 74.996) (end 135.916 80) (width 0.762) (layer F.Cu) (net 24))
 (segment (start 140.92 73.58) (end 140.92 74.996) (width 0.762) (layer F.Cu) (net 24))
 (segment (start 129.54 80) (end 133.04 76.5) (width 0.762) (layer F.Cu) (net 21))
 (segment (start 129 80) (end 129.54 80) (width 0.762) (layer F.Cu) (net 21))
 (segment (start 83.79032 61.46) (end 90.5 61.46) (width 0.762) (layer F.Cu) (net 9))
 (segment (start 83.5 61.75032) (end 83.79032 61.46) (width 0.762) (layer F.Cu) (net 9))
 (segment (start 82.24968 60.5) (end 83.5 61.75032) (width 0.762) (layer F.Cu) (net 9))
 (segment (start 78 60.5) (end 82.24968 60.5) (width 0.762) (layer F.Cu) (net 9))
 (segment (start 115.865641 103) (end 116.220141 103.3545) (width 0.762) (layer F.Cu) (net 1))
 (segment (start 113.114641 109) (end 116.220141 105.8945) (width 0.762) (layer F.Cu) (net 12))
 (segment (start 106 111) (end 108 109) (width 0.762) (layer F.Cu) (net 12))
 (segment (start 108 109) (end 113.114641 109) (width 0.762) (layer F.Cu) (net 12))
 (segment (start 135.666793 111) (end 134.49936 111) (width 0.762) (layer F.Cu) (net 23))
 (segment (start 136.916 111) (end 135.666793 111) (width 0.762) (layer F.Cu) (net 23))
 (segment (start 141.1 106.816) (end 136.916 111) (width 0.762) (layer F.Cu) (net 23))
 (segment (start 141.1 105.4) (end 141.1 106.816) (width 0.762) (layer F.Cu) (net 23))
 (segment (start 130 111) (end 133 108) (width 0.762) (layer F.Cu) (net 19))
 (segment (start 129.50064 111) (end 130 111) (width 0.762) (layer F.Cu) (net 19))
 (segment (start 82.5 78.4) (end 82.5 81) (width 0.762) (layer F.Cu) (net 22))
 (segment (start 89.4 71.5) (end 82.5 78.4) (width 0.762) (layer F.Cu) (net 22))
 (segment (start 108.96 67.5) (end 93.4 67.5) (width 0.762) (layer F.Cu) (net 22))
 (segment (start 93.4 67.5) (end 89.4 71.5) (width 0.762) (layer F.Cu) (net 22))
 (segment (start 82.5 88.6) (end 93.6 88.6) (width 0.762) (layer F.Cu) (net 20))
 (segment (start 82.5 86) (end 82.5 88.6) (width 0.762) (layer F.Cu) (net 20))
 (segment (start 98.549949 88.6) (end 93.6 88.6) (width 0.762) (layer F.Cu) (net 20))
 (segment (start 107.96 98.010051) (end 98.549949 88.6) (width 0.762) (layer F.Cu) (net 20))
 (segment (start 107.96 99) (end 107.96 98.010051) (width 0.762) (layer F.Cu) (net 20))
 (segment (start 123.6 76.5) (end 123.32 76.78) (width 0.762) (layer F.Cu) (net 18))
 (segment (start 130.5 76.5) (end 123.6 76.5) (width 0.762) (layer F.Cu) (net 18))
 (segment (start 124.274641 108) (end 123.840141 108.4345) (width 0.762) (layer F.Cu) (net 14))
 (segment (start 130.46 108) (end 124.274641 108) (width 0.762) (layer F.Cu) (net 14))
 (segment (start 123.32 79.32) (end 123.32 80.45137) (width 0.762) (layer F.Cu) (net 15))
 (segment (start 120.96 82.81137) (end 120.96 92.5) (width 0.762) (layer F.Cu) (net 15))
 (segment (start 123.32 80.45137) (end 120.96 82.81137) (width 0.762) (layer F.Cu) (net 15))
 (segment (start 115.7 84.7) (end 115.88 84.88) (width 0.762) (layer F.Cu) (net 17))
 (segment (start 115.7 79.32) (end 115.7 84.7) (width 0.762) (layer F.Cu) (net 17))
 (segment (start 123.840141 110.9745) (end 123.840141 114.159859) (width 0.762) (layer F.Cu) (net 11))
 (segment (start 121.54 116.46) (end 121.54 125.31) (width 0.762) (layer F.Cu) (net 11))
 (segment (start 123.840141 114.159859) (end 121.54 116.46) (width 0.762) (layer F.Cu) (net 11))
 (segment (start 116.220141 117.450141) (end 116.46 117.69) (width 0.762) (layer F.Cu) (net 13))
 (segment (start 116.220141 110.9745) (end 116.220141 117.450141) (width 0.762) (layer F.Cu) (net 13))
 (segment (start 86 105.04) (end 85.77 104.81) (width 0.762) (layer F.Cu) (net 5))
 (segment (start 83.23 102.27) (end 85.77 104.81) (width 0.762) (layer F.Cu) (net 5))
 (segment (start 83.23 97.19) (end 83.23 102.27) (width 0.762) (layer F.Cu) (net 5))
 (segment (start 85.77 119.77) (end 86.42 120.42) (width 0.762) (layer F.Cu) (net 5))
 (segment (start 85.77 104.81) (end 85.77 119.77) (width 0.762) (layer F.Cu) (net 5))
 (segment (start 94.73 104.81) (end 96.5 103.04) (width 0.762) (layer F.Cu) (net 8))
 (segment (start 88.31 104.81) (end 94.73 104.81) (width 0.762) (layer F.Cu) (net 8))
 (segment (start 124.08 124.052765) (end 121.527235 121.5) (width 0.762) (layer B.Cu) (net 8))
 (segment (start 124.08 125.31) (end 124.08 124.052765) (width 0.762) (layer B.Cu) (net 8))
 (segment (start 97.199999 111.199999) (end 107.5 121.5) (width 0.762) (layer B.Cu) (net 8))
 (segment (start 97.199999 103.739999) (end 97.199999 111.199999) (width 0.762) (layer B.Cu) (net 8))
 (segment (start 121.527235 121.5) (end 107.5 121.5) (width 0.762) (layer B.Cu) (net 8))
 (segment (start 96.5 103.04) (end 97.199999 103.739999) (width 0.762) (layer B.Cu) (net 8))
 (segment (start 107.5 121.5) (end 107.46 121.5) (width 0.762) (layer B.Cu) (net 8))
 (segment (start 80.69 95.932765) (end 81.622765 95) (width 0.762) (layer F.Cu) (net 7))
 (segment (start 80.69 97.19) (end 80.69 95.932765) (width 0.762) (layer F.Cu) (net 7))
 (segment (start 81.622765 95) (end 85.5 95) (width 0.762) (layer F.Cu) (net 7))
 (segment (start 91 95) (end 96.5 100.5) (width 0.762) (layer F.Cu) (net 7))
 (segment (start 85.5 95) (end 91 95) (width 0.762) (layer F.Cu) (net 7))
 (segment (start 96.5 98) (end 96.5 100.5) (width 0.762) (layer B.Cu) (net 7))
 (segment (start 99 95.5) (end 96.5 98) (width 0.762) (layer B.Cu) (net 7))
 (segment (start 122.5 95.5) (end 99 95.5) (width 0.762) (layer B.Cu) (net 7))
 (segment (start 123.5 92.5) (end 123.5 94.5) (width 0.762) (layer B.Cu) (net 7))
 (segment (start 123.5 94.5) (end 122.5 95.5) (width 0.762) (layer B.Cu) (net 7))
 (segment (start 110.5 102.00064) (end 110.99936 102.5) (width 0.762) (layer F.Cu) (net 2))
 (segment (start 110.5 99) (end 110.5 102.00064) (width 0.762) (layer F.Cu) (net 2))
 (segment (start 109.50128 102.5) (end 106.00128 106) (width 0.762) (layer F.Cu) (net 2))
 (segment (start 110.99936 102.5) (end 109.50128 102.5) (width 0.762) (layer F.Cu) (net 2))
 (segment (start 114.138 71.7) (end 112.5 73.338) (width 0.762) (layer F.Cu) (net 3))
 (segment (start 115.7 71.7) (end 114.138 71.7) (width 0.762) (layer F.Cu) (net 3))
 (segment (start 111.662 73.338) (end 111.5 73.5) (width 0.762) (layer F.Cu) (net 3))
 (segment (start 112.5 73.338) (end 111.662 73.338) (width 0.762) (layer F.Cu) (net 3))
 (segment (start 113.6455 103.3545) (end 116.220141 103.3545) (width 0.762) (layer F.Cu) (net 1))
 (segment (start 111 106) (end 113.6455 103.3545) (width 0.762) (layer F.Cu) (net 1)))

